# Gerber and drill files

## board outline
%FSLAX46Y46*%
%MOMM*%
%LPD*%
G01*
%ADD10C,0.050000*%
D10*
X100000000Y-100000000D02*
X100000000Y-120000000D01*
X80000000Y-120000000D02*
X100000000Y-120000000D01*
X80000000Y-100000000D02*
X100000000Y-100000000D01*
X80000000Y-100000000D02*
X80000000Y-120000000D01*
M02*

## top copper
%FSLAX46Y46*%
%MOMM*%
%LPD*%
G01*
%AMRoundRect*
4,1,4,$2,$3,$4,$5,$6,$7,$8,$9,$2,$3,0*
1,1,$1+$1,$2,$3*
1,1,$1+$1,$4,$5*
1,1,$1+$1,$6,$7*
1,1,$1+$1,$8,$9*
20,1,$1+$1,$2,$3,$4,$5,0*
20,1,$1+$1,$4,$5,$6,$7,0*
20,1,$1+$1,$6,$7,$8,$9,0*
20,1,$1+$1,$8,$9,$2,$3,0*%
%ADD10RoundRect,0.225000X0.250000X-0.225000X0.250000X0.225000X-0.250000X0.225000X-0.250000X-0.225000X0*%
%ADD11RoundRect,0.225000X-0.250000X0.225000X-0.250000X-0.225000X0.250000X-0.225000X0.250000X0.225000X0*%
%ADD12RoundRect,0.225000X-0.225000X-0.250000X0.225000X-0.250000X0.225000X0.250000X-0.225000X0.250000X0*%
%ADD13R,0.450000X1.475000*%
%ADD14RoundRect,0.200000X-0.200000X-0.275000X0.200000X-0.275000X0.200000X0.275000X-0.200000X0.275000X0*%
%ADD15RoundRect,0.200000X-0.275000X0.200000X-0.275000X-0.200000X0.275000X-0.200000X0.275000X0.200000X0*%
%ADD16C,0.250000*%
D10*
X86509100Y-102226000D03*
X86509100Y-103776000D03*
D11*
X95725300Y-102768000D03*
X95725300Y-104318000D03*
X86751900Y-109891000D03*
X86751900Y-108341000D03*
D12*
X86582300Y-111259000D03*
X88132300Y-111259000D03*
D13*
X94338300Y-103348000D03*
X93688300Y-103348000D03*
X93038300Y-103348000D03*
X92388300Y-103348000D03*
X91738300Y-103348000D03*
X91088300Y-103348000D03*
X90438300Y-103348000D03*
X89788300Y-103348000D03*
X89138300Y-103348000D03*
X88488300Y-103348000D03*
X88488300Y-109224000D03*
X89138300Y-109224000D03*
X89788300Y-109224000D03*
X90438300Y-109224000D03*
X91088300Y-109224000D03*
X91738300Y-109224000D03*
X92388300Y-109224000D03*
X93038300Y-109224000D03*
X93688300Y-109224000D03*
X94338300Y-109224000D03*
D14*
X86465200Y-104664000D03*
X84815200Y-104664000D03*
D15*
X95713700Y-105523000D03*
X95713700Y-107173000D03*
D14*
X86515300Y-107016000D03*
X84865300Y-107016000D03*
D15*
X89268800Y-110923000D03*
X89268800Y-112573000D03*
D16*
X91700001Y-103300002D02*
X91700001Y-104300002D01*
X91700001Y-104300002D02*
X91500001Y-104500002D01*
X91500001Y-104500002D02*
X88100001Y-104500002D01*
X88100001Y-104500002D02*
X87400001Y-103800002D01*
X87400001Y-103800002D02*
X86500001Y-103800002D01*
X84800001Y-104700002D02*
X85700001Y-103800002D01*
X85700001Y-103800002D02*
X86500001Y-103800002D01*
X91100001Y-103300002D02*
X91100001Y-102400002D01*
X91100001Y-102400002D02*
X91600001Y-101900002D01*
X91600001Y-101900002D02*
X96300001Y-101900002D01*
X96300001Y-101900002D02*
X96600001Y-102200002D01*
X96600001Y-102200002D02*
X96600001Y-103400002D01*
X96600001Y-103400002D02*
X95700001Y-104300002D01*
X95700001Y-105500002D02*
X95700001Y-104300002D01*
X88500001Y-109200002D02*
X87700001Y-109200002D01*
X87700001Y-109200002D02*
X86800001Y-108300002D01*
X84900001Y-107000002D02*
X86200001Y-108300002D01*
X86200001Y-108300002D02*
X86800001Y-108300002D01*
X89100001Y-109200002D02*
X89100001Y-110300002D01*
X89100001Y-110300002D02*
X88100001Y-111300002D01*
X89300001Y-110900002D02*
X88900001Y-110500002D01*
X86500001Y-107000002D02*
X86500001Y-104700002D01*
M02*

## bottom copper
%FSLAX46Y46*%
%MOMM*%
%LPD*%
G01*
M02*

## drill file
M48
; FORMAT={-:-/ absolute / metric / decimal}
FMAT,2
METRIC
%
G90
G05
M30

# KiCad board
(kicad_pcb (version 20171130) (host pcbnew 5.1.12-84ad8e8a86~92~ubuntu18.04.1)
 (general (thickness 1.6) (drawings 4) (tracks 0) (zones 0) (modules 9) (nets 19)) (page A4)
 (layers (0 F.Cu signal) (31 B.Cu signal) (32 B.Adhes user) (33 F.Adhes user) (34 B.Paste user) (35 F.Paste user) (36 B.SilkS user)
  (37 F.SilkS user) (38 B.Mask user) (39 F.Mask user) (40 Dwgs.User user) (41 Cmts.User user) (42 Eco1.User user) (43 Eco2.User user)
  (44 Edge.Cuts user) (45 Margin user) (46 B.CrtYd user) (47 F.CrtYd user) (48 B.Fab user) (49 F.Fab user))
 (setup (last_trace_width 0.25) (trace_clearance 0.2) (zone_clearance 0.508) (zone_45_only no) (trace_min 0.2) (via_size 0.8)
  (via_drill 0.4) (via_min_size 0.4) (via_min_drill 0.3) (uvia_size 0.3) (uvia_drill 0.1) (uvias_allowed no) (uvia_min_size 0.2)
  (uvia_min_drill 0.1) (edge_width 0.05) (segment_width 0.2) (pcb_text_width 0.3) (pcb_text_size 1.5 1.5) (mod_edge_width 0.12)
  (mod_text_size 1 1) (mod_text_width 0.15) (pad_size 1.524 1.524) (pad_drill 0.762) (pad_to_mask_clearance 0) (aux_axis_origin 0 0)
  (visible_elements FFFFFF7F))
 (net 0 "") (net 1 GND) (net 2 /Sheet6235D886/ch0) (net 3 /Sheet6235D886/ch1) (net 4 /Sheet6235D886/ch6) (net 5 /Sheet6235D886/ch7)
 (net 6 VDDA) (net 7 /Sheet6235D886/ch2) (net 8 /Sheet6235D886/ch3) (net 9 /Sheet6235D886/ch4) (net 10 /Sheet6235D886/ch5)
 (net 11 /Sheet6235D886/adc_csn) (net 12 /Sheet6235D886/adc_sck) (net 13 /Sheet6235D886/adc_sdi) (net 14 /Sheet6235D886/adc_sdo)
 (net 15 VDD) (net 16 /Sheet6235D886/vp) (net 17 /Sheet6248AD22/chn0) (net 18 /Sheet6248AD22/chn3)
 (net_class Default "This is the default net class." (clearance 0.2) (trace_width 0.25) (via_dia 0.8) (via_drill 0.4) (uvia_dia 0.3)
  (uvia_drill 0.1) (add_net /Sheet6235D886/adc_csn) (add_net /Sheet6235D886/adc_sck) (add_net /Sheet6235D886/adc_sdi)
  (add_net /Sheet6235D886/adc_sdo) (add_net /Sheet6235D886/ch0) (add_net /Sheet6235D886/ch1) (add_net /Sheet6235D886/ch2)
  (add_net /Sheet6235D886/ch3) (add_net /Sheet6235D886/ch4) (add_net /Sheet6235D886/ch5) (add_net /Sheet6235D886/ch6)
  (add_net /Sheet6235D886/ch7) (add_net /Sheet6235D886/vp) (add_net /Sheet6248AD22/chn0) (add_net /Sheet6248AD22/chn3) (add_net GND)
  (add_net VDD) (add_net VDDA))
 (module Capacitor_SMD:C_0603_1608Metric (layer F.Cu) (at 86.509100 103.001000 90.000000)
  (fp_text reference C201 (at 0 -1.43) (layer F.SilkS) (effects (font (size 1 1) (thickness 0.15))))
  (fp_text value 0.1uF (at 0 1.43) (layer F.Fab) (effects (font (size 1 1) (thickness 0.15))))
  (pad 2 smd roundrect (at 0.775 0 90.000000) (size 0.9 0.95) (layers F.Cu F.Mask F.Paste) (roundrect_rratio 0.25) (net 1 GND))
  (pad 1 smd roundrect (at -0.775 0 90.000000) (size 0.9 0.95) (layers F.Cu F.Mask F.Paste) (roundrect_rratio 0.25)
   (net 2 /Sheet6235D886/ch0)))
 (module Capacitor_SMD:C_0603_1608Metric (layer F.Cu) (at 95.725300 103.543000 270.000000)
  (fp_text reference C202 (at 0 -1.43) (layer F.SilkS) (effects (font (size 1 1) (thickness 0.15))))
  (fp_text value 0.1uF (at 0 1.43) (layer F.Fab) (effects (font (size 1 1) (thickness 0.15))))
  (pad 1 smd roundrect (at -0.775 0 270.000000) (size 0.9 0.95) (layers F.Cu F.Mask F.Paste) (roundrect_rratio 0.25) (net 1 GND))
  (pad 2 smd roundrect (at 0.775 0 270.000000) (size 0.9 0.95) (layers F.Cu F.Mask F.Paste) (roundrect_rratio 0.25)
   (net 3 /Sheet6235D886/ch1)))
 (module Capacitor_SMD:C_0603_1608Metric (layer F.Cu) (at 86.751900 109.116000 270.000000)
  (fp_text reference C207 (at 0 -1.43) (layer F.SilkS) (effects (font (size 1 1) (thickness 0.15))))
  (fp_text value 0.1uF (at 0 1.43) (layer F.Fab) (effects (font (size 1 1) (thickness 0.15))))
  (pad 2 smd roundrect (at 0.775 0 270.000000) (size 0.9 0.95) (layers F.Cu F.Mask F.Paste) (roundrect_rratio 0.25) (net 1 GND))
  (pad 1 smd roundrect (at -0.775 0 270.000000) (size 0.9 0.95) (layers F.Cu F.Mask F.Paste) (roundrect_rratio 0.25)
   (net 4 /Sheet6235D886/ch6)))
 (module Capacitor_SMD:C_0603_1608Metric (layer F.Cu) (at 87.357300 111.259000)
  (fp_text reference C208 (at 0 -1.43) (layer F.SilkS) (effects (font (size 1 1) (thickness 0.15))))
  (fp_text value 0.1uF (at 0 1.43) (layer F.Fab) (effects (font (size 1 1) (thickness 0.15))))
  (pad 1 smd roundrect (at -0.775 0) (size 0.9 0.95) (layers F.Cu F.Mask F.Paste) (roundrect_rratio 0.25) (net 1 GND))
  (pad 2 smd roundrect (at 0.775 0) (size 0.9 0.95) (layers F.Cu F.Mask F.Paste) (roundrect_rratio 0.25) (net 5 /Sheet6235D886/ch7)))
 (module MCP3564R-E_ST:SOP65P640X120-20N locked (layer F.Cu) (at 91.413300 106.286000 270.000000)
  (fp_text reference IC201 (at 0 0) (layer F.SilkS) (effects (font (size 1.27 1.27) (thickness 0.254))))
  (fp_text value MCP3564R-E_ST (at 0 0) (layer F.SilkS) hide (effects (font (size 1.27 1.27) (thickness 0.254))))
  (pad 1 smd rect (at -2.938 -2.925) (size 0.45 1.475) (layers F.Cu F.Mask F.Paste) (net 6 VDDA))
  (pad 2 smd rect (at -2.938 -2.275) (size 0.45 1.475) (layers F.Cu F.Mask F.Paste) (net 1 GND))
  (pad 3 smd rect (at -2.938 -1.625) (size 0.45 1.475) (layers F.Cu F.Mask F.Paste) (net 1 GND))
  (pad 4 smd rect (at -2.938 -0.975) (size 0.45 1.475) (layers F.Cu F.Mask F.Paste))
  (pad 5 smd rect (at -2.938 -0.325) (size 0.45 1.475) (layers F.Cu F.Mask F.Paste) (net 2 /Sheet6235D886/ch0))
  (pad 6 smd rect (at -2.938 0.325) (size 0.45 1.475) (layers F.Cu F.Mask F.Paste) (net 3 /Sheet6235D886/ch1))
  (pad 7 smd rect (at -2.938 0.975) (size 0.45 1.475) (layers F.Cu F.Mask F.Paste) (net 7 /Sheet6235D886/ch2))
  (pad 8 smd rect (at -2.938 1.625) (size 0.45 1.475) (layers F.Cu F.Mask F.Paste) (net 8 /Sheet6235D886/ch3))
  (pad 9 smd rect (at -2.938 2.275) (size 0.45 1.475) (layers F.Cu F.Mask F.Paste) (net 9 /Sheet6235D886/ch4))
  (pad 10 smd rect (at -2.938 2.925) (size 0.45 1.475) (layers F.Cu F.Mask F.Paste) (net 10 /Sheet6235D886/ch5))
  (pad 11 smd rect (at 2.938 2.925) (size 0.45 1.475) (layers F.Cu F.Mask F.Paste) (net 4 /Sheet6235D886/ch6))
  (pad 12 smd rect (at 2.938 2.275) (size 0.45 1.475) (layers F.Cu F.Mask F.Paste) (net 5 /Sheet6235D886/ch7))
  (pad 13 smd rect (at 2.938 1.625) (size 0.45 1.475) (layers F.Cu F.Mask F.Paste) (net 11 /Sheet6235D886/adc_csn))
  (pad 14 smd rect (at 2.938 0.975) (size 0.45 1.475) (layers F.Cu F.Mask F.Paste) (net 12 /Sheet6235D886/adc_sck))
  (pad 15 smd rect (at 2.938 0.325) (size 0.45 1.475) (layers F.Cu F.Mask F.Paste) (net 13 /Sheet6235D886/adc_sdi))
  (pad 16 smd rect (at 2.938 -0.325) (size 0.45 1.475) (layers F.Cu F.Mask F.Paste) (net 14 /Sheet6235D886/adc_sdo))
  (pad 17 smd rect (at 2.938 -0.975) (size 0.45 1.475) (layers F.Cu F.Mask F.Paste))
  (pad 18 smd rect (at 2.938 -1.625) (size 0.45 1.475) (layers F.Cu F.Mask F.Paste))
  (pad 19 smd rect (at 2.938 -2.275) (size 0.45 1.475) (layers F.Cu F.Mask F.Paste) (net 1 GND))
  (pad 20 smd rect (at 2.938 -2.925) (size 0.45 1.475) (layers F.Cu F.Mask F.Paste) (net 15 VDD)))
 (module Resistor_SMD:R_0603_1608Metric (layer F.Cu) (at 85.640200 104.664000)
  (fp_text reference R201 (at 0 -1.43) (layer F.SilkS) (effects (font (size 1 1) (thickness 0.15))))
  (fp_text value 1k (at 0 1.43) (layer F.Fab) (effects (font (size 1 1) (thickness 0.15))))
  (pad 2 smd roundrect (at 0.825 0) (size 0.8 0.95) (layers F.Cu F.Mask F.Paste) (roundrect_rratio 0.25) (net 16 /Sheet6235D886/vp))
  (pad 1 smd roundrect (at -0.825 0) (size 0.8 0.95) (layers F.Cu F.Mask F.Paste) (roundrect_rratio 0.25) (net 2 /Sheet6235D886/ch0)))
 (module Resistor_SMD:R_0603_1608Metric (layer F.Cu) (at 95.713700 106.348000 270.000000)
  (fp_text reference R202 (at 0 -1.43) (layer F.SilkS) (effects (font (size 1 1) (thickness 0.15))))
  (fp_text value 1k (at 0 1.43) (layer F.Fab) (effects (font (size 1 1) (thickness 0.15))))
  (pad 1 smd roundrect (at -0.825 0 270.000000) (size 0.8 0.95) (layers F.Cu F.Mask F.Paste) (roundrect_rratio 0.25)
   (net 3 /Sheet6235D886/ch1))
  (pad 2 smd roundrect (at 0.825 0 270.000000) (size 0.8 0.95) (layers F.Cu F.Mask F.Paste) (roundrect_rratio 0.25)
   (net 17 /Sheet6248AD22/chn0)))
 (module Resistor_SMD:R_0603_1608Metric (layer F.Cu) (at 85.690300 107.016000)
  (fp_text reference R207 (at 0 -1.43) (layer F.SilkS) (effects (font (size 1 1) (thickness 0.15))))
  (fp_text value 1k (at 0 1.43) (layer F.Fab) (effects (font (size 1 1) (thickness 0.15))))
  (pad 2 smd roundrect (at 0.825 0) (size 0.8 0.95) (layers F.Cu F.Mask F.Paste) (roundrect_rratio 0.25) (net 16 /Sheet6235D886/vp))
  (pad 1 smd roundrect (at -0.825 0) (size 0.8 0.95) (layers F.Cu F.Mask F.Paste) (roundrect_rratio 0.25) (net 4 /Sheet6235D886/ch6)))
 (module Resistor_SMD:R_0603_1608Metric (layer F.Cu) (at 89.268800 111.748000 270.000000)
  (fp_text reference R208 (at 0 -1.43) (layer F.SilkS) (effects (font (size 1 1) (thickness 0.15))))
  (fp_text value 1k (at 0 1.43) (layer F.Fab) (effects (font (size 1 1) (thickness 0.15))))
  (pad 1 smd roundrect (at -0.825 0 270.000000) (size 0.8 0.95) (layers F.Cu F.Mask F.Paste) (roundrect_rratio 0.25)
   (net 5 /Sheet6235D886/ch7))
  (pad 2 smd roundrect (at 0.825 0 270.000000) (size 0.8 0.95) (layers F.Cu F.Mask F.Paste) (roundrect_rratio 0.25)
   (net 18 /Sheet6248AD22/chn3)))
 (gr_line (start 100 100) (end 100 120) (layer Edge.Cuts) (width 0.05))
 (gr_line (start 80 120) (end 100 120) (layer Edge.Cuts) (width 0.05))
 (gr_line (start 80 100) (end 100 100) (layer Edge.Cuts) (width 0.05))
 (gr_line (start 80 100) (end 80 120) (layer Edge.Cuts) (width 0.05))
 (segment (start 91.700001 103.300002) (end 91.700001 104.300002) (width 0.250000) (layer F.Cu) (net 2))
 (segment (start 91.700001 104.300002) (end 91.500001 104.500002) (width 0.250000) (layer F.Cu) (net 2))
 (segment (start 91.500001 104.500002) (end 88.100001 104.500002) (width 0.250000) (layer F.Cu) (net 2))
 (segment (start 88.100001 104.500002) (end 87.400001 103.800002) (width 0.250000) (layer F.Cu) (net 2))
 (segment (start 87.400001 103.800002) (end 86.500001 103.800002) (width 0.250000) (layer F.Cu) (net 2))
 (segment (start 84.800001 104.700002) (end 85.700001 103.800002) (width 0.250000) (layer F.Cu) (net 2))
 (segment (start 85.700001 103.800002) (end 86.500001 103.800002) (width 0.250000) (layer F.Cu) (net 2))
 (segment (start 91.100001 103.300002) (end 91.100001 102.400002) (width 0.250000) (layer F.Cu) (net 3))
 (segment (start 91.100001 102.400002) (end 91.600001 101.900002) (width 0.250000) (layer F.Cu) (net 3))
 (segment (start 91.600001 101.900002) (end 96.300001 101.900002) (width 0.250000) (layer F.Cu) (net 3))
 (segment (start 96.300001 101.900002) (end 96.600001 102.200002) (width 0.250000) (layer F.Cu) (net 3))
 (segment (start 96.600001 102.200002) (end 96.600001 103.400002) (width 0.250000) (layer F.Cu) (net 3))
 (segment (start 96.600001 103.400002) (end 95.700001 104.300002) (width 0.250000) (layer F.Cu) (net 3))
 (segment (start 95.700001 105.500002) (end 95.700001 104.300002) (width 0.250000) (layer F.Cu) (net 3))
 (segment (start 88.500001 109.200002) (end 87.700001 109.200002) (width 0.250000) (layer F.Cu) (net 4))
 (segment (start 87.700001 109.200002) (end 86.800001 108.300002) (width 0.250000) (layer F.Cu) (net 4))
 (segment (start 84.900001 107.000002) (end 86.200001 108.300002) (width 0.250000) (layer F.Cu) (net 4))
 (segment (start 86.200001 108.300002) (end 86.800001 108.300002) (width 0.250000) (layer F.Cu) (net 4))
 (segment (start 89.100001 109.200002) (end 89.100001 110.300002) (width 0.250000) (layer F.Cu) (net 5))
 (segment (start 89.100001 110.300002) (end 88.100001 111.300002) (width 0.250000) (layer F.Cu) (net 5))
 (segment (start 89.300001 110.900002) (end 88.900001 110.500002) (width 0.250000) (layer F.Cu) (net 5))
 (segment (start 86.500001 107.000002) (end 86.500001 104.700002) (width 0.250000) (layer F.Cu) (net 16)))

